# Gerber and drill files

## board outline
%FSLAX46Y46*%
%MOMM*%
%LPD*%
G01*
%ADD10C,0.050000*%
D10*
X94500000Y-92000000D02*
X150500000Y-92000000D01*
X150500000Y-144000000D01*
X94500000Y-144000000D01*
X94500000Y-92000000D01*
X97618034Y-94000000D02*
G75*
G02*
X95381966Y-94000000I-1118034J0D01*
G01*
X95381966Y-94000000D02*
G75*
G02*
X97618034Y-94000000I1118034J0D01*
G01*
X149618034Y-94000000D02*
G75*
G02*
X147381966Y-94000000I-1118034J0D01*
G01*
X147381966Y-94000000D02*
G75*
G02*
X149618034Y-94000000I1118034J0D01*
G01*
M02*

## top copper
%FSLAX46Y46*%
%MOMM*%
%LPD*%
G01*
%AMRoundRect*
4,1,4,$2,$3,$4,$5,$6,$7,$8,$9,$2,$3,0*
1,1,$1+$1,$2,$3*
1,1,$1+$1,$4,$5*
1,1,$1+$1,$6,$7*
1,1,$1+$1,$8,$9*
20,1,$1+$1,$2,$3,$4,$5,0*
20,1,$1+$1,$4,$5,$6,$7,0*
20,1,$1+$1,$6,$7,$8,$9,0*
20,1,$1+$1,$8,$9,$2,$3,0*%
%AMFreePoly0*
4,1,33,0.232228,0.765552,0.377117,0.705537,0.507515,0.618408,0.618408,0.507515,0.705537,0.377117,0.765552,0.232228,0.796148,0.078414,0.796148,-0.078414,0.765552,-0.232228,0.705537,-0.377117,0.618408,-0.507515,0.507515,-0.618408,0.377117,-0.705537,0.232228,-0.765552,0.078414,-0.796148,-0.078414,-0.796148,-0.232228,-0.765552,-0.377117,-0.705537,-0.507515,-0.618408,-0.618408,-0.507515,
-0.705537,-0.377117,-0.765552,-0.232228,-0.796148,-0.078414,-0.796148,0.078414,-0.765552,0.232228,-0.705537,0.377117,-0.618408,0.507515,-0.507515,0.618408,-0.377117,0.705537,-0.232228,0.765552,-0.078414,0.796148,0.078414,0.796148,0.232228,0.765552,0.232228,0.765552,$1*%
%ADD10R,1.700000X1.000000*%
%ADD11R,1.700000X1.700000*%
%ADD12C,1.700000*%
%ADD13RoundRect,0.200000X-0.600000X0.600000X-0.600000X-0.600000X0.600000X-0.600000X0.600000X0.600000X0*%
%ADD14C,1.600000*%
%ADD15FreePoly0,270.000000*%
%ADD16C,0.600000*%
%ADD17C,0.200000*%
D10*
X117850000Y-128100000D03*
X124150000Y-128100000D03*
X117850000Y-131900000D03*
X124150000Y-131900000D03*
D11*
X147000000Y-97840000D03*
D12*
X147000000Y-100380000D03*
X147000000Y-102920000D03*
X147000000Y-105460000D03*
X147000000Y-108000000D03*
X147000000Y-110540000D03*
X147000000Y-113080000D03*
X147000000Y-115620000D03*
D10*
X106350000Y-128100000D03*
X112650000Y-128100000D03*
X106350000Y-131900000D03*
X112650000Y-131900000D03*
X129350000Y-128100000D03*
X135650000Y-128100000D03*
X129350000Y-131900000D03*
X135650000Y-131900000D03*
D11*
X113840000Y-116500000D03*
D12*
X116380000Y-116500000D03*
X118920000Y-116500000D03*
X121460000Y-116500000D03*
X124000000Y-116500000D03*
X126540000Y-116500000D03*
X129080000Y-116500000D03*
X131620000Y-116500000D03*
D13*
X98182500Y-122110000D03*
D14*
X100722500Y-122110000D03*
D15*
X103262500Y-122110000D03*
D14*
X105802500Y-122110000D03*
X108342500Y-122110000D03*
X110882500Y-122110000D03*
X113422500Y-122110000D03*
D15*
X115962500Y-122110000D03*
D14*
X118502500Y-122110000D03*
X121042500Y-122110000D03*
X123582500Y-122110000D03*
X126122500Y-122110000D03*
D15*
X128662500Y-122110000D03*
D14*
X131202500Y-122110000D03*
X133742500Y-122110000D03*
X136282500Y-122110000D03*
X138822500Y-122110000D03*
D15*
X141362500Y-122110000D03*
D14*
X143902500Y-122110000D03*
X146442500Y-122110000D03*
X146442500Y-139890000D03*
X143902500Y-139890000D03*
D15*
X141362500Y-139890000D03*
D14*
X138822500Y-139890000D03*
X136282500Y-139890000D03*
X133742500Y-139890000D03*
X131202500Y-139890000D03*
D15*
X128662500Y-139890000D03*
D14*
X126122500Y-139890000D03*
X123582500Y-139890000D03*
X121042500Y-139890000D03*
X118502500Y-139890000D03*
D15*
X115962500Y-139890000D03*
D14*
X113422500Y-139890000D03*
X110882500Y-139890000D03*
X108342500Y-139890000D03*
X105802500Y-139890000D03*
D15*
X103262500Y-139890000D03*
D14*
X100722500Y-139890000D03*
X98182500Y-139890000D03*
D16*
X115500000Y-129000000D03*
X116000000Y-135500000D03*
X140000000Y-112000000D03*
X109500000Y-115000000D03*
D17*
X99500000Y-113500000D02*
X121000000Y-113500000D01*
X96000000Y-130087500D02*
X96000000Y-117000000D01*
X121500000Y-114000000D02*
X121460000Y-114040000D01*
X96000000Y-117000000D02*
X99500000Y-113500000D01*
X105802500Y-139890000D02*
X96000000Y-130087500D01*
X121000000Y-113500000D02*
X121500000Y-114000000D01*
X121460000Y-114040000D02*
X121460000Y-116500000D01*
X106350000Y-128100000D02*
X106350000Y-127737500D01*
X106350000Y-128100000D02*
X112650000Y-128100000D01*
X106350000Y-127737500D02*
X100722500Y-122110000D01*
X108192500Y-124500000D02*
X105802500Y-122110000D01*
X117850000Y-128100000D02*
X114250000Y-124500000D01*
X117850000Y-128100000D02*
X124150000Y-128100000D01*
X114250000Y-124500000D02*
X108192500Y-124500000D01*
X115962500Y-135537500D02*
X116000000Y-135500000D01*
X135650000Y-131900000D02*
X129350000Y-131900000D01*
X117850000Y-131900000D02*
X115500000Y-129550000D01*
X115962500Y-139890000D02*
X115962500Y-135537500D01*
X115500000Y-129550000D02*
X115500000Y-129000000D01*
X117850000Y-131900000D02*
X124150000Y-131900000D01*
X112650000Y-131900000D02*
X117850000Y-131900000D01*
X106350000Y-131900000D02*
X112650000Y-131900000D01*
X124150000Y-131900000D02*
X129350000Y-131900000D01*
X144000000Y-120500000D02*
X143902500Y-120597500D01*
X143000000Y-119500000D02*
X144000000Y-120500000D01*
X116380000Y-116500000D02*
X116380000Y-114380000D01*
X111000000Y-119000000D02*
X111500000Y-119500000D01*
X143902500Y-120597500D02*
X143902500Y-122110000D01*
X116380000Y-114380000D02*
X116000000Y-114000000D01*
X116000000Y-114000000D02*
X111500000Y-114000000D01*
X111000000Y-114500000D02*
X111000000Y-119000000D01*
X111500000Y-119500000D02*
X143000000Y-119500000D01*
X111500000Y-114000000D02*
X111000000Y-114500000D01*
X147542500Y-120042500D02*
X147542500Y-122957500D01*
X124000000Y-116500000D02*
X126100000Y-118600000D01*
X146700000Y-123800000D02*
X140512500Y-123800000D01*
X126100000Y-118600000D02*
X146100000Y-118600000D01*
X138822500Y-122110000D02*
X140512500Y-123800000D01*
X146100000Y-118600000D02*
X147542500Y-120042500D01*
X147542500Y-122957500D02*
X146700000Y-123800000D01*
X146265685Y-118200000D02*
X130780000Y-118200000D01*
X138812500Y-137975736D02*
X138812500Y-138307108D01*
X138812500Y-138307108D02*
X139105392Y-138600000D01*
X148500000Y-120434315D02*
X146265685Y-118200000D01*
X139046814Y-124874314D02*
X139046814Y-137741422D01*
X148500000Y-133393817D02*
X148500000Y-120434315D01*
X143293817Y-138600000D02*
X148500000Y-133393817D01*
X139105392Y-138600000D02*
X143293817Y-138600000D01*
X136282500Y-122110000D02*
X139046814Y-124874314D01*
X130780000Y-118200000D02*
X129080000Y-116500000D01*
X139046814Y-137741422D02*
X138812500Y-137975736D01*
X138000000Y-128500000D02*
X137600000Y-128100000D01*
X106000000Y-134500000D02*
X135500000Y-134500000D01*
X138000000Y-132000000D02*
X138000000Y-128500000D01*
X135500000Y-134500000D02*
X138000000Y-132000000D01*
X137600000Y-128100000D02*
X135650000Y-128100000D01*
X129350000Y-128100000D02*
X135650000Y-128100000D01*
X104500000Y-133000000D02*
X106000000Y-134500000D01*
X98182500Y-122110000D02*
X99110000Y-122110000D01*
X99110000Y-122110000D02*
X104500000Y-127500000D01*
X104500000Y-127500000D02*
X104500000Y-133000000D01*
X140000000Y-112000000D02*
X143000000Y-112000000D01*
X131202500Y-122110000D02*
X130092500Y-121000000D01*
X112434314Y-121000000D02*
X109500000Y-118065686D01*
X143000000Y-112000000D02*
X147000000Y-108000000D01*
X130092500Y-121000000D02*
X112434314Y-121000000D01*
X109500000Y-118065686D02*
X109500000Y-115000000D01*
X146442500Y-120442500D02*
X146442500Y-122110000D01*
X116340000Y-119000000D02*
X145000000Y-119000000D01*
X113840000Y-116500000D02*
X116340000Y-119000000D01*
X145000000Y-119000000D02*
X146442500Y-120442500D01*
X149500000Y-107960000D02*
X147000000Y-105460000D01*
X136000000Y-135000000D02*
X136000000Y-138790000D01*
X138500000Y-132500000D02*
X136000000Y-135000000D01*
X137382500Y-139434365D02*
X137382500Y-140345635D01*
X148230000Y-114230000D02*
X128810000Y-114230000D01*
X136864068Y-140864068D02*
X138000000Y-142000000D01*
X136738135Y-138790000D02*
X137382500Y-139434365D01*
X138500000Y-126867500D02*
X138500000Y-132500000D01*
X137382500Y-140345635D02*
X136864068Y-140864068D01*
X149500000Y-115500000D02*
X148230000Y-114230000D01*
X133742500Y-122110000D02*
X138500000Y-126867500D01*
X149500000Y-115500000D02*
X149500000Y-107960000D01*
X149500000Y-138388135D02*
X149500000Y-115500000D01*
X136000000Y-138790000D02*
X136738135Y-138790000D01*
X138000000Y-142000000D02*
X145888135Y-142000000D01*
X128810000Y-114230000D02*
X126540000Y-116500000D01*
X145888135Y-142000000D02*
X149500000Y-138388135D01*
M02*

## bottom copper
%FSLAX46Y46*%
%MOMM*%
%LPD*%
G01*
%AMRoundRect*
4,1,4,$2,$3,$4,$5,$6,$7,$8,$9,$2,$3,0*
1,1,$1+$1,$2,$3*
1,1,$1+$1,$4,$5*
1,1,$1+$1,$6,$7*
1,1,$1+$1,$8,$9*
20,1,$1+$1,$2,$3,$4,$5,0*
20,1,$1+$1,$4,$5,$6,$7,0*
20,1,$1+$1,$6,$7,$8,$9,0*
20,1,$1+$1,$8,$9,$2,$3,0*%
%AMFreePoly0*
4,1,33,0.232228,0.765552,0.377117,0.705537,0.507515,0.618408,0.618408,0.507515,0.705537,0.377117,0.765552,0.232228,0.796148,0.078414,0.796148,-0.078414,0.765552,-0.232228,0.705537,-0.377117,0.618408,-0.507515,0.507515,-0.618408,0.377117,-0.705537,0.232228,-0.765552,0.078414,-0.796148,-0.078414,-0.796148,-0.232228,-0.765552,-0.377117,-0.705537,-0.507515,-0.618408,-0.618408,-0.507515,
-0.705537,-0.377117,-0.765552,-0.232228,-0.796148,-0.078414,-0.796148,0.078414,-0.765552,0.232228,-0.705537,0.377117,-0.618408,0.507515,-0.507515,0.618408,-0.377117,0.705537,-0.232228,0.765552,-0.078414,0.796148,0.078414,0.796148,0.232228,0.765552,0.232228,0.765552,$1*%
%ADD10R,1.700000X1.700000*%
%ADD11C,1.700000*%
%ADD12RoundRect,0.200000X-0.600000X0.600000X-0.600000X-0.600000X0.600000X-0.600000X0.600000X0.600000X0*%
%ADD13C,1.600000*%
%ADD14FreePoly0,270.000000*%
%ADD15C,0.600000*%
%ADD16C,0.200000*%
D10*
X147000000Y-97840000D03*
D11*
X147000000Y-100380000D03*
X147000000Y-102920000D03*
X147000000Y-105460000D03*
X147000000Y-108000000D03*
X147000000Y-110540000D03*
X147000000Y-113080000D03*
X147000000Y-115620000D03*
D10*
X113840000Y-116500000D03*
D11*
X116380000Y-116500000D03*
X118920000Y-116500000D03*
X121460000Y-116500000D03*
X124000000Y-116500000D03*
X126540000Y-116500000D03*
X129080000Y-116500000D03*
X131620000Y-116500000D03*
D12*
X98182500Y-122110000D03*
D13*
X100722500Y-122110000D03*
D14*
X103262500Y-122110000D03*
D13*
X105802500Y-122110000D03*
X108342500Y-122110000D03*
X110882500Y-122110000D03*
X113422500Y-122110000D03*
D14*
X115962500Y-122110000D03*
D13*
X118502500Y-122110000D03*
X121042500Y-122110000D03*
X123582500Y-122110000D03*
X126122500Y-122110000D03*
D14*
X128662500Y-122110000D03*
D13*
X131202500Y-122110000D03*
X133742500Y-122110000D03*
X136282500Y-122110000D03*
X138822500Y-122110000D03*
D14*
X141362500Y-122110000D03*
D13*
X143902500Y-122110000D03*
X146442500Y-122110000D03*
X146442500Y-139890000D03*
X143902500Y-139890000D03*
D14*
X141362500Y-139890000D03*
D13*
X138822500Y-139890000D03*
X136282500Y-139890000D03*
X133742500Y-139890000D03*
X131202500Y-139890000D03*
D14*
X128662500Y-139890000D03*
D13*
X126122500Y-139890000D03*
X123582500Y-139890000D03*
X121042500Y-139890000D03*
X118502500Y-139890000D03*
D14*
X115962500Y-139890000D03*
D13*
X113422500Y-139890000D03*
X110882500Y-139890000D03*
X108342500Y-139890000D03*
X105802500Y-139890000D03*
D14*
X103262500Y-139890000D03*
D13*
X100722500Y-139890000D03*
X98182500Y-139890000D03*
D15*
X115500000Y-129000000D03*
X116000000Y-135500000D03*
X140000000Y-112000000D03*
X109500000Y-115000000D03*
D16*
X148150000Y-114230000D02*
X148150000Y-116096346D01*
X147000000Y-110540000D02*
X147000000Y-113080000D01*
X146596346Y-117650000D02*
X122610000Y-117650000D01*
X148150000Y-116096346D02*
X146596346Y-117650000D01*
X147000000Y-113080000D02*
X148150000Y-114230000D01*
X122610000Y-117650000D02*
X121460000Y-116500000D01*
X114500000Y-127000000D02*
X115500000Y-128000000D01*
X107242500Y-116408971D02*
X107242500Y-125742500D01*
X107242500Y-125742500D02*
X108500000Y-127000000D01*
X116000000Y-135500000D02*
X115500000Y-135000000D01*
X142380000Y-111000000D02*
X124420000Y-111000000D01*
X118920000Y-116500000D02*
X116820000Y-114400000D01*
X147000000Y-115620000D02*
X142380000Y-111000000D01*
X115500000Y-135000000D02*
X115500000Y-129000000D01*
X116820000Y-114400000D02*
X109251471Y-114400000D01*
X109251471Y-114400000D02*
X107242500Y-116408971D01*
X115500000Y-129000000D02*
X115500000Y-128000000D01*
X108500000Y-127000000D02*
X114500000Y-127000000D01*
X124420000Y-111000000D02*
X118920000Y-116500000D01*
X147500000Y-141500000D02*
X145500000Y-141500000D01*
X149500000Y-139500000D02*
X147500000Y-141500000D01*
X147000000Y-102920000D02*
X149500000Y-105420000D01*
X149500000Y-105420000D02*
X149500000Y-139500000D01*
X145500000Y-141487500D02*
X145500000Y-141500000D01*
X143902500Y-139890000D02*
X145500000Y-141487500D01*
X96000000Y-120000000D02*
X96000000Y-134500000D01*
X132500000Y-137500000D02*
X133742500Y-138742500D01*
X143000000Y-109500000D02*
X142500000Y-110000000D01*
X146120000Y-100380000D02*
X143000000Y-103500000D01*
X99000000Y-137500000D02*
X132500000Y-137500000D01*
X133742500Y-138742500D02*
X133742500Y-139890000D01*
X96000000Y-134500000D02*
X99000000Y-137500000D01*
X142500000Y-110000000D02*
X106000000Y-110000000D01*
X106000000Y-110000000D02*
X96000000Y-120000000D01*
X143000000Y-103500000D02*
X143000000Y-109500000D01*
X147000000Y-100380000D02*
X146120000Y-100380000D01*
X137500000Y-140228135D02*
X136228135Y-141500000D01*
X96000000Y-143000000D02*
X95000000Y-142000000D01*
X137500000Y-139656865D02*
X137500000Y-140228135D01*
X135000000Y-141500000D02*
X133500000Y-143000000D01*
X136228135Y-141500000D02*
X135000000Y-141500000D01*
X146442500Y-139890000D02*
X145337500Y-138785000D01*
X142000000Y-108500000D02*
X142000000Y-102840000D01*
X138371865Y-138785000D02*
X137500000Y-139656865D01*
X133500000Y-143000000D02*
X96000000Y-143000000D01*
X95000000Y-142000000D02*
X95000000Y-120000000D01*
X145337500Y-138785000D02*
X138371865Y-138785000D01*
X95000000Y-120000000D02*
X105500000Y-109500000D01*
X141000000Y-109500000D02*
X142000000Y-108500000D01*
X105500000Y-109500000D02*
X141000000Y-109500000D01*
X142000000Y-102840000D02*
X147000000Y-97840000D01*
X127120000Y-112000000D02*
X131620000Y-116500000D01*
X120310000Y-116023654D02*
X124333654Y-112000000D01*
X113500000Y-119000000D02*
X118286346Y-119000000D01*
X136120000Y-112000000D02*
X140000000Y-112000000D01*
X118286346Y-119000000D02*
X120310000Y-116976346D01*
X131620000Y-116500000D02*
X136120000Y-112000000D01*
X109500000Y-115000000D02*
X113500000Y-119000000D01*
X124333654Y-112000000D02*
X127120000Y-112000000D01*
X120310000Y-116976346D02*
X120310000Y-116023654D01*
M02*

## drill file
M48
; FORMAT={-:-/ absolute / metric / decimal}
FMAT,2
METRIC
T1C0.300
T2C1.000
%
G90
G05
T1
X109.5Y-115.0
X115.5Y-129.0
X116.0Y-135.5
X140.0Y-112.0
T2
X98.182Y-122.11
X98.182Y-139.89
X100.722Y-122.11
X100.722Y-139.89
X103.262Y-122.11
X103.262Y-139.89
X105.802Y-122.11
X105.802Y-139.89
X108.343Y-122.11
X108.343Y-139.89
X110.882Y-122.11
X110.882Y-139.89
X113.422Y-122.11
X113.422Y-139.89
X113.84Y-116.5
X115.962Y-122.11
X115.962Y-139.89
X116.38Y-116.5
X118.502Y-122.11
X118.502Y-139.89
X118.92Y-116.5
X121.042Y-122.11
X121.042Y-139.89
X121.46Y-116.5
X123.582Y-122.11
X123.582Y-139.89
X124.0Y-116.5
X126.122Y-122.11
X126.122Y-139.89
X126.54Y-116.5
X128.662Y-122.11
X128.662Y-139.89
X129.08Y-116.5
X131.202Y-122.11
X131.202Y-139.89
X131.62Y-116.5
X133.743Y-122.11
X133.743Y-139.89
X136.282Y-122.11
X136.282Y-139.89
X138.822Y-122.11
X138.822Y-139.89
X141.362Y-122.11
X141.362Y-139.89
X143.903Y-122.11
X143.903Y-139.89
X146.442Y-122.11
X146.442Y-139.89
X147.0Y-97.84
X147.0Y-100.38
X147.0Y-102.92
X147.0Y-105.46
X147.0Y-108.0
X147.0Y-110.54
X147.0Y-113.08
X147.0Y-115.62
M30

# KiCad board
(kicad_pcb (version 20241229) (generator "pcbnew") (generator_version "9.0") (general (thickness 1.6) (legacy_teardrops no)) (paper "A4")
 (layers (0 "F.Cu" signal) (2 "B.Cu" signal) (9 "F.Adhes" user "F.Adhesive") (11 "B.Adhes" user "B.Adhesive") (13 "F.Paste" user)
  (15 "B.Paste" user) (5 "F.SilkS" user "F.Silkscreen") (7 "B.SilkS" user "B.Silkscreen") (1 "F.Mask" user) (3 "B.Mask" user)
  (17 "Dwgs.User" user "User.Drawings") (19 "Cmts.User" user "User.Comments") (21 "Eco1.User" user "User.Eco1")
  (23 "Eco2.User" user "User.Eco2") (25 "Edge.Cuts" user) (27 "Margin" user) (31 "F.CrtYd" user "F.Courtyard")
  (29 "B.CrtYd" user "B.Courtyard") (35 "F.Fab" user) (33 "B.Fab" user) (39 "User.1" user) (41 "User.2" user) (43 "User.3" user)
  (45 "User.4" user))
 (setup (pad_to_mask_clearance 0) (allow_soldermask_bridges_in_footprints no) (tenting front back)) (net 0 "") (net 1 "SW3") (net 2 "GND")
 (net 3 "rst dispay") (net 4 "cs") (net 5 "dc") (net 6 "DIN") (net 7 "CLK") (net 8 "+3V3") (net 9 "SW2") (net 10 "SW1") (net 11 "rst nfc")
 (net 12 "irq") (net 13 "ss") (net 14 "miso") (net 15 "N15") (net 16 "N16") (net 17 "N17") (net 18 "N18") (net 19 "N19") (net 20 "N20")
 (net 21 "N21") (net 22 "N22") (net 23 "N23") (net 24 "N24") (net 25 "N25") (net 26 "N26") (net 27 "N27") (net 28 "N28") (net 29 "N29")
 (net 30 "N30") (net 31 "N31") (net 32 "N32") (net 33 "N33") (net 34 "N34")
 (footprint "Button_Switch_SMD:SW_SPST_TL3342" (layer "F.Cu") (at 121 130)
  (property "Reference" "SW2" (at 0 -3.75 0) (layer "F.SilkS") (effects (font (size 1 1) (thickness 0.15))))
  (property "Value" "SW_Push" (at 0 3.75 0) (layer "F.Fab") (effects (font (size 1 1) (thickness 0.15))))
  (pad "1" smd rect (at -3.15 -1.9) (size 1.7 1) (layers "F.Cu" "F.Mask" "F.Paste") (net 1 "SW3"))
  (pad "1" smd rect (at 3.15 -1.9) (size 1.7 1) (layers "F.Cu" "F.Mask" "F.Paste") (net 1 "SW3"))
  (pad "2" smd rect (at -3.15 1.9) (size 1.7 1) (layers "F.Cu" "F.Mask" "F.Paste") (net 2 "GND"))
  (pad "2" smd rect (at 3.15 1.9) (size 1.7 1) (layers "F.Cu" "F.Mask" "F.Paste") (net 2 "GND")))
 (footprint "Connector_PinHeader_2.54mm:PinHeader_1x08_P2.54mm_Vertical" (layer "F.Cu") (at 147 97.84)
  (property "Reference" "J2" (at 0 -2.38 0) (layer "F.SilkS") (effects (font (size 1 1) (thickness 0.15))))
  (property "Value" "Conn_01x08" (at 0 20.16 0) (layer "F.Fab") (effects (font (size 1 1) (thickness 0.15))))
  (pad "1" thru_hole rect (at 0 0) (size 1.7 1.7) (drill 1) (layers "*.Cu" "*.Mask") (remove_unused_layers no) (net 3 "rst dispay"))
  (pad "2" thru_hole circle (at 0 2.54) (size 1.7 1.7) (drill 1) (layers "*.Cu" "*.Mask") (remove_unused_layers no) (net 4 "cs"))
  (pad "3" thru_hole circle (at 0 5.08) (size 1.7 1.7) (drill 1) (layers "*.Cu" "*.Mask") (remove_unused_layers no) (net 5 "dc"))
  (pad "4" thru_hole circle (at 0 7.62) (size 1.7 1.7) (drill 1) (layers "*.Cu" "*.Mask") (remove_unused_layers no) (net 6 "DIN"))
  (pad "5" thru_hole circle (at 0 10.16) (size 1.7 1.7) (drill 1) (layers "*.Cu" "*.Mask") (remove_unused_layers no) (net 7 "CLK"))
  (pad "6" thru_hole circle (at 0 12.7) (size 1.7 1.7) (drill 1) (layers "*.Cu" "*.Mask") (remove_unused_layers no) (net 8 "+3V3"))
  (pad "7" thru_hole circle (at 0 15.24) (size 1.7 1.7) (drill 1) (layers "*.Cu" "*.Mask") (remove_unused_layers no) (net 8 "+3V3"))
  (pad "8" thru_hole circle (at 0 17.78) (size 1.7 1.7) (drill 1) (layers "*.Cu" "*.Mask") (remove_unused_layers no) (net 2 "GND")))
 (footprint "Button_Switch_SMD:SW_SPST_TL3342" (layer "F.Cu") (at 109.5 130)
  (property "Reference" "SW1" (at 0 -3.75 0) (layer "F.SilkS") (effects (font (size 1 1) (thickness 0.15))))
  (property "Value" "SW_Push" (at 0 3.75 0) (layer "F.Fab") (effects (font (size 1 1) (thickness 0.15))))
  (pad "1" smd rect (at -3.15 -1.9) (size 1.7 1) (layers "F.Cu" "F.Mask" "F.Paste") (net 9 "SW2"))
  (pad "1" smd rect (at 3.15 -1.9) (size 1.7 1) (layers "F.Cu" "F.Mask" "F.Paste") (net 9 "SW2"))
  (pad "2" smd rect (at -3.15 1.9) (size 1.7 1) (layers "F.Cu" "F.Mask" "F.Paste") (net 2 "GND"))
  (pad "2" smd rect (at 3.15 1.9) (size 1.7 1) (layers "F.Cu" "F.Mask" "F.Paste") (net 2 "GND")))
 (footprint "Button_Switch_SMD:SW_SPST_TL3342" (layer "F.Cu") (at 132.5 130)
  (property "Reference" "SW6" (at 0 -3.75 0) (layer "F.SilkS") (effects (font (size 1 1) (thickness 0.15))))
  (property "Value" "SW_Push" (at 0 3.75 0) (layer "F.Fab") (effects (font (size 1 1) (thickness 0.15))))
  (pad "1" smd rect (at -3.15 -1.9) (size 1.7 1) (layers "F.Cu" "F.Mask" "F.Paste") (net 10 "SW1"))
  (pad "1" smd rect (at 3.15 -1.9) (size 1.7 1) (layers "F.Cu" "F.Mask" "F.Paste") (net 10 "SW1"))
  (pad "2" smd rect (at -3.15 1.9) (size 1.7 1) (layers "F.Cu" "F.Mask" "F.Paste") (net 2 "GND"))
  (pad "2" smd rect (at 3.15 1.9) (size 1.7 1) (layers "F.Cu" "F.Mask" "F.Paste") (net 2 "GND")))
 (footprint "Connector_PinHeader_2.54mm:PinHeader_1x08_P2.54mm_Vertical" (layer "F.Cu") (at 113.84 116.5 90)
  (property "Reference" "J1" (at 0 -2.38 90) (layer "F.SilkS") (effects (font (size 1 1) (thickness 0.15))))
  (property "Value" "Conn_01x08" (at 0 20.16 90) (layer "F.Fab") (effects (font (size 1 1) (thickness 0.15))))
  (pad "1" thru_hole rect (at 0 0 90) (size 1.7 1.7) (drill 1) (layers "*.Cu" "*.Mask") (remove_unused_layers no) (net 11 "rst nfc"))
  (pad "2" thru_hole circle (at 0 2.54 90) (size 1.7 1.7) (drill 1) (layers "*.Cu" "*.Mask") (remove_unused_layers no) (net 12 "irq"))
  (pad "3" thru_hole circle (at 0 5.08 90) (size 1.7 1.7) (drill 1) (layers "*.Cu" "*.Mask") (remove_unused_layers no) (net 2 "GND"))
  (pad "4" thru_hole circle (at 0 7.62 90) (size 1.7 1.7) (drill 1) (layers "*.Cu" "*.Mask") (remove_unused_layers no) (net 8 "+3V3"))
  (pad "5" thru_hole circle (at 0 10.16 90) (size 1.7 1.7) (drill 1) (layers "*.Cu" "*.Mask") (remove_unused_layers no) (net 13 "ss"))
  (pad "6" thru_hole circle (at 0 12.7 90) (size 1.7 1.7) (drill 1) (layers "*.Cu" "*.Mask") (remove_unused_layers no) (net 6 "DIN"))
  (pad "7" thru_hole circle (at 0 15.24 90) (size 1.7 1.7) (drill 1) (layers "*.Cu" "*.Mask") (remove_unused_layers no) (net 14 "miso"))
  (pad "8" thru_hole circle (at 0 17.78 90) (size 1.7 1.7) (drill 1) (layers "*.Cu" "*.Mask") (remove_unused_layers no) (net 7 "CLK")))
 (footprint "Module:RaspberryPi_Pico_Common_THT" (layer "B.Cu") (at 98.1825 122.11 -90)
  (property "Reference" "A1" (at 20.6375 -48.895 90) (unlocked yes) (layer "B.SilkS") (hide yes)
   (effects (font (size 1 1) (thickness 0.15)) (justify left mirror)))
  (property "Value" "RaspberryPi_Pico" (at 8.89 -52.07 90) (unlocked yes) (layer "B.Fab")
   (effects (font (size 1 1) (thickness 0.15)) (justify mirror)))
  (pad "1" thru_hole roundrect (at 0 0 270) (size 1.6 1.6) (drill 1) (layers "*.Cu" "*.Mask") (remove_unused_layers no)
   (roundrect_rratio 0.125) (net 10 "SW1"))
  (pad "2" thru_hole circle (at 0 -2.54 270) (size 1.6 1.6) (drill 1) (layers "*.Cu" "*.Mask") (remove_unused_layers no) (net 9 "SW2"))
  (pad "3" thru_hole custom (at 0 -5.08 270) (size 1.6 1.6) (drill 1) (layers "*.Cu" "*.Mask") (remove_unused_layers no) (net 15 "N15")
   (options (clearance outline) (anchor circle)) (primitives))
  (pad "4" thru_hole circle (at 0 -7.62 270) (size 1.6 1.6) (drill 1) (layers "*.Cu" "*.Mask") (remove_unused_layers no) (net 1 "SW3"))
  (pad "5" thru_hole circle (at 0 -10.16 270) (size 1.6 1.6) (drill 1) (layers "*.Cu" "*.Mask") (remove_unused_layers no) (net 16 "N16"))
  (pad "6" thru_hole circle (at 0 -12.7 270) (size 1.6 1.6) (drill 1) (layers "*.Cu" "*.Mask") (remove_unused_layers no) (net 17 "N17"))
  (pad "7" thru_hole circle (at 0 -15.24 270) (size 1.6 1.6) (drill 1) (layers "*.Cu" "*.Mask") (remove_unused_layers no) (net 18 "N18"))
  (pad "8" thru_hole custom (at 0 -17.78 270) (size 1.6 1.6) (drill 1) (layers "*.Cu" "*.Mask") (remove_unused_layers no) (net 15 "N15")
   (options (clearance outline) (anchor circle)) (primitives))
  (pad "9" thru_hole circle (at 0 -20.32 270) (size 1.6 1.6) (drill 1) (layers "*.Cu" "*.Mask") (remove_unused_layers no) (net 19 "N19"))
  (pad "10" thru_hole circle (at 0 -22.86 270) (size 1.6 1.6) (drill 1) (layers "*.Cu" "*.Mask") (remove_unused_layers no) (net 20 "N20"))
  (pad "11" thru_hole circle (at 0 -25.4 270) (size 1.6 1.6) (drill 1) (layers "*.Cu" "*.Mask") (remove_unused_layers no) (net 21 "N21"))
  (pad "12" thru_hole circle (at 0 -27.94 270) (size 1.6 1.6) (drill 1) (layers "*.Cu" "*.Mask") (remove_unused_layers no) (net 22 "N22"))
  (pad "13" thru_hole custom (at 0 -30.48 270) (size 1.6 1.6) (drill 1) (layers "*.Cu" "*.Mask") (remove_unused_layers no) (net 15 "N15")
   (options (clearance outline) (anchor circle)) (primitives))
  (pad "14" thru_hole circle (at 0 -33.02 270) (size 1.6 1.6) (drill 1) (layers "*.Cu" "*.Mask") (remove_unused_layers no) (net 7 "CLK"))
  (pad "15" thru_hole circle (at 0 -35.56 270) (size 1.6 1.6) (drill 1) (layers "*.Cu" "*.Mask") (remove_unused_layers no) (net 6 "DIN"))
  (pad "16" thru_hole circle (at 0 -38.1 270) (size 1.6 1.6) (drill 1) (layers "*.Cu" "*.Mask") (remove_unused_layers no) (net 14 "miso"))
  (pad "17" thru_hole circle (at 0 -40.64 270) (size 1.6 1.6) (drill 1) (layers "*.Cu" "*.Mask") (remove_unused_layers no) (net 13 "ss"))
  (pad "18" thru_hole custom (at 0 -43.18 270) (size 1.6 1.6) (drill 1) (layers "*.Cu" "*.Mask") (remove_unused_layers no) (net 15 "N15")
   (options (clearance outline) (anchor circle)) (primitives))
  (pad "19" thru_hole circle (at 0 -45.72 270) (size 1.6 1.6) (drill 1) (layers "*.Cu" "*.Mask") (remove_unused_layers no) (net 12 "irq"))
  (pad "20" thru_hole circle (at 0 -48.26 270) (size 1.6 1.6) (drill 1) (layers "*.Cu" "*.Mask") (remove_unused_layers no)
   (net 11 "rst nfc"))
  (pad "21" thru_hole circle (at 17.78 -48.26 270) (size 1.6 1.6) (drill 1) (layers "*.Cu" "*.Mask") (remove_unused_layers no)
   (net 3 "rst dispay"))
  (pad "22" thru_hole circle (at 17.78 -45.72 270) (size 1.6 1.6) (drill 1) (layers "*.Cu" "*.Mask") (remove_unused_layers no) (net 5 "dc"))
  (pad "23" thru_hole custom (at 17.78 -43.18 270) (size 1.6 1.6) (drill 1) (layers "*.Cu" "*.Mask") (remove_unused_layers no)
   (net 15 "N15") (options (clearance outline) (anchor circle)) (primitives))
  (pad "24" thru_hole circle (at 17.78 -40.64 270) (size 1.6 1.6) (drill 1) (layers "*.Cu" "*.Mask") (remove_unused_layers no)
   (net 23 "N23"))
  (pad "25" thru_hole circle (at 17.78 -38.1 270) (size 1.6 1.6) (drill 1) (layers "*.Cu" "*.Mask") (remove_unused_layers no) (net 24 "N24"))
  (pad "26" thru_hole circle (at 17.78 -35.56 270) (size 1.6 1.6) (drill 1) (layers "*.Cu" "*.Mask") (remove_unused_layers no) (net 4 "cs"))
  (pad "27" thru_hole circle (at 17.78 -33.02 270) (size 1.6 1.6) (drill 1) (layers "*.Cu" "*.Mask") (remove_unused_layers no)
   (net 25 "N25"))
  (pad "28" thru_hole custom (at 17.78 -30.48 270) (size 1.6 1.6) (drill 1) (layers "*.Cu" "*.Mask") (remove_unused_layers no)
   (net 15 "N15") (options (clearance outline) (anchor circle)) (primitives))
  (pad "29" thru_hole circle (at 17.78 -27.94 270) (size 1.6 1.6) (drill 1) (layers "*.Cu" "*.Mask") (remove_unused_layers no)
   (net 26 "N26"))
  (pad "30" thru_hole circle (at 17.78 -25.4 270) (size 1.6 1.6) (drill 1) (layers "*.Cu" "*.Mask") (remove_unused_layers no) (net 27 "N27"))
  (pad "31" thru_hole circle (at 17.78 -22.86 270) (size 1.6 1.6) (drill 1) (layers "*.Cu" "*.Mask") (remove_unused_layers no)
   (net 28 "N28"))
  (pad "32" thru_hole circle (at 17.78 -20.32 270) (size 1.6 1.6) (drill 1) (layers "*.Cu" "*.Mask") (remove_unused_layers no)
   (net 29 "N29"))
  (pad "33" thru_hole custom (at 17.78 -17.78 270) (size 1.6 1.6) (drill 1) (layers "*.Cu" "*.Mask") (remove_unused_layers no) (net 2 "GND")
   (options (clearance outline) (anchor circle)) (primitives))
  (pad "34" thru_hole circle (at 17.78 -15.24 270) (size 1.6 1.6) (drill 1) (layers "*.Cu" "*.Mask") (remove_unused_layers no)
   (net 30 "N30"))
  (pad "35" thru_hole circle (at 17.78 -12.7 270) (size 1.6 1.6) (drill 1) (layers "*.Cu" "*.Mask") (remove_unused_layers no) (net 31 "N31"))
  (pad "36" thru_hole circle (at 17.78 -10.16 270) (size 1.6 1.6) (drill 1) (layers "*.Cu" "*.Mask") (remove_unused_layers no)
   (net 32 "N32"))
  (pad "37" thru_hole circle (at 17.78 -7.62 270) (size 1.6 1.6) (drill 1) (layers "*.Cu" "*.Mask") (remove_unused_layers no) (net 8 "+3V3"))
  (pad "38" thru_hole custom (at 17.78 -5.08 270) (size 1.6 1.6) (drill 1) (layers "*.Cu" "*.Mask") (remove_unused_layers no) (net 15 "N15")
   (options (clearance outline) (anchor circle)) (primitives))
  (pad "39" thru_hole circle (at 17.78 -2.54 270) (size 1.6 1.6) (drill 1) (layers "*.Cu" "*.Mask") (remove_unused_layers no) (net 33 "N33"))
  (pad "40" thru_hole circle (at 17.78 0 270) (size 1.6 1.6) (drill 1) (layers "*.Cu" "*.Mask") (remove_unused_layers no) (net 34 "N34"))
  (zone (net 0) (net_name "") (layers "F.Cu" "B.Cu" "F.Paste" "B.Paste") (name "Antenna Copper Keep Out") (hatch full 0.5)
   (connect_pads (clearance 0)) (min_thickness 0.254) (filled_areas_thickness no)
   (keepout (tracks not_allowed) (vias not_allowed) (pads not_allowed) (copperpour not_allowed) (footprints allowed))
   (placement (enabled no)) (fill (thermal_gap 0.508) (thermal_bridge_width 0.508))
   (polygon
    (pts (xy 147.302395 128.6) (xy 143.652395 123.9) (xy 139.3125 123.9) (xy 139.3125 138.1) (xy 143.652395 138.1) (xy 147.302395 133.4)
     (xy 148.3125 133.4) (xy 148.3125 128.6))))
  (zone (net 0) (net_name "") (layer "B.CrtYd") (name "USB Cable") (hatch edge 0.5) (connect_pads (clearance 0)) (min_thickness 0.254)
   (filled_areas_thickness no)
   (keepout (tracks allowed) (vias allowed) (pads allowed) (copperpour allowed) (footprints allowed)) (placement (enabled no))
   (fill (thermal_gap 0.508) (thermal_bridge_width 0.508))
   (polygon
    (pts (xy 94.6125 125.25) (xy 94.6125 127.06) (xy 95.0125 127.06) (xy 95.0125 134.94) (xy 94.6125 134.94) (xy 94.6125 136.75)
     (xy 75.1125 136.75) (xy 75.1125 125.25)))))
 (gr_rect (start 94.5 92) (end 150.5 144) (stroke (width 0.05) (type default)) (fill no) (layer "Edge.Cuts"))
 (gr_circle (center 96.5 94) (end 97.5 94.5) (stroke (width 0.05) (type default)) (fill no) (layer "Edge.Cuts"))
 (gr_circle (center 148.5 94) (end 149.5 94.5) (stroke (width 0.05) (type default)) (fill no) (layer "Edge.Cuts"))
 (segment (start 99.5 113.5) (end 121 113.5) (width 0.2) (layer "F.Cu") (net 8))
 (segment (start 96 130.0875) (end 96 117) (width 0.2) (layer "F.Cu") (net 8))
 (segment (start 121.5 114) (end 121.46 114.04) (width 0.2) (layer "F.Cu") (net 8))
 (segment (start 96 117) (end 99.5 113.5) (width 0.2) (layer "F.Cu") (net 8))
 (segment (start 105.8025 139.89) (end 96 130.0875) (width 0.2) (layer "F.Cu") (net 8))
 (segment (start 121 113.5) (end 121.5 114) (width 0.2) (layer "F.Cu") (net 8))
 (segment (start 121.46 114.04) (end 121.46 116.5) (width 0.2) (layer "F.Cu") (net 8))
 (segment (start 148.15 114.23) (end 148.15 116.096346) (width 0.2) (layer "B.Cu") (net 8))
 (segment (start 147 110.54) (end 147 113.08) (width 0.2) (layer "B.Cu") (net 8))
 (segment (start 146.596346 117.65) (end 122.61 117.65) (width 0.2) (layer "B.Cu") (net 8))
 (segment (start 148.15 116.096346) (end 146.596346 117.65) (width 0.2) (layer "B.Cu") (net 8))
 (segment (start 147 113.08) (end 148.15 114.23) (width 0.2) (layer "B.Cu") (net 8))
 (segment (start 122.61 117.65) (end 121.46 116.5) (width 0.2) (layer "B.Cu") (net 8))
 (segment (start 106.35 128.1) (end 106.35 127.7375) (width 0.2) (layer "F.Cu") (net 9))
 (segment (start 106.35 128.1) (end 112.65 128.1) (width 0.2) (layer "F.Cu") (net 9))
 (segment (start 106.35 127.7375) (end 100.7225 122.11) (width 0.2) (layer "F.Cu") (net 9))
 (segment (start 108.1925 124.5) (end 105.8025 122.11) (width 0.2) (layer "F.Cu") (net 1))
 (segment (start 117.85 128.1) (end 114.25 124.5) (width 0.2) (layer "F.Cu") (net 1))
 (segment (start 117.85 128.1) (end 124.15 128.1) (width 0.2) (layer "F.Cu") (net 1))
 (segment (start 114.25 124.5) (end 108.1925 124.5) (width 0.2) (layer "F.Cu") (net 1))
 (segment (start 115.9625 135.5375) (end 116 135.5) (width 0.2) (layer "F.Cu") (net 2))
 (segment (start 135.65 131.9) (end 129.35 131.9) (width 0.2) (layer "F.Cu") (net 2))
 (segment (start 117.85 131.9) (end 115.5 129.55) (width 0.2) (layer "F.Cu") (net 2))
 (segment (start 115.9625 139.89) (end 115.9625 135.5375) (width 0.2) (layer "F.Cu") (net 2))
 (segment (start 115.5 129.55) (end 115.5 129) (width 0.2) (layer "F.Cu") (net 2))
 (segment (start 117.85 131.9) (end 124.15 131.9) (width 0.2) (layer "F.Cu") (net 2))
 (segment (start 112.65 131.9) (end 117.85 131.9) (width 0.2) (layer "F.Cu") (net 2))
 (segment (start 106.35 131.9) (end 112.65 131.9) (width 0.2) (layer "F.Cu") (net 2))
 (segment (start 124.15 131.9) (end 129.35 131.9) (width 0.2) (layer "F.Cu") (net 2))
 (via (at 115.5 129) (size 0.6) (drill 0.3) (layers "F.Cu" "B.Cu") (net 2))
 (via (at 116 135.5) (size 0.6) (drill 0.3) (layers "F.Cu" "B.Cu") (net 2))
 (segment (start 114.5 127) (end 115.5 128) (width 0.2) (layer "B.Cu") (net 2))
 (segment (start 107.2425 116.408971) (end 107.2425 125.7425) (width 0.2) (layer "B.Cu") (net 2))
 (segment (start 107.2425 125.7425) (end 108.5 127) (width 0.2) (layer "B.Cu") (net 2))
 (segment (start 116 135.5) (end 115.5 135) (width 0.2) (layer "B.Cu") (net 2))
 (segment (start 142.38 111) (end 124.42 111) (width 0.2) (layer "B.Cu") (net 2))
 (segment (start 118.92 116.5) (end 116.82 114.4) (width 0.2) (layer "B.Cu") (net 2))
 (segment (start 147 115.62) (end 142.38 111) (width 0.2) (layer "B.Cu") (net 2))
 (segment (start 115.5 135) (end 115.5 129) (width 0.2) (layer "B.Cu") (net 2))
 (segment (start 116.82 114.4) (end 109.251471 114.4) (width 0.2) (layer "B.Cu") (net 2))
 (segment (start 109.251471 114.4) (end 107.2425 116.408971) (width 0.2) (layer "B.Cu") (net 2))
 (segment (start 115.5 129) (end 115.5 128) (width 0.2) (layer "B.Cu") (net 2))
 (segment (start 108.5 127) (end 114.5 127) (width 0.2) (layer "B.Cu") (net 2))
 (segment (start 124.42 111) (end 118.92 116.5) (width 0.2) (layer "B.Cu") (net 2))
 (segment (start 144 120.5) (end 143.9025 120.5975) (width 0.2) (layer "F.Cu") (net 12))
 (segment (start 143 119.5) (end 144 120.5) (width 0.2) (layer "F.Cu") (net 12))
 (segment (start 116.38 116.5) (end 116.38 114.38) (width 0.2) (layer "F.Cu") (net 12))
 (segment (start 111 119) (end 111.5 119.5) (width 0.2) (layer "F.Cu") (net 12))
 (segment (start 143.9025 120.5975) (end 143.9025 122.11) (width 0.2) (layer "F.Cu") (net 12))
 (segment (start 116.38 114.38) (end 116 114) (width 0.2) (layer "F.Cu") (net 12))
 (segment (start 116 114) (end 111.5 114) (width 0.2) (layer "F.Cu") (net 12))
 (segment (start 111 114.5) (end 111 119) (width 0.2) (layer "F.Cu") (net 12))
 (segment (start 111.5 119.5) (end 143 119.5) (width 0.2) (layer "F.Cu") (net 12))
 (segment (start 111.5 114) (end 111 114.5) (width 0.2) (layer "F.Cu") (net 12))
 (segment (start 147.5 141.5) (end 145.5 141.5) (width 0.2) (layer "B.Cu") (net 5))
 (segment (start 149.5 139.5) (end 147.5 141.5) (width 0.2) (layer "B.Cu") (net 5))
 (segment (start 147 102.92) (end 149.5 105.42) (width 0.2) (layer "B.Cu") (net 5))
 (segment (start 149.5 105.42) (end 149.5 139.5) (width 0.2) (layer "B.Cu") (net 5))
 (segment (start 145.5 141.4875) (end 145.5 141.5) (width 0.2) (layer "B.Cu") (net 5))
 (segment (start 143.9025 139.89) (end 145.5 141.4875) (width 0.2) (layer "B.Cu") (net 5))
 (segment (start 147.5425 120.0425) (end 147.5425 122.9575) (width 0.2) (layer "F.Cu") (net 13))
 (segment (start 124 116.5) (end 126.1 118.6) (width 0.2) (layer "F.Cu") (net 13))
 (segment (start 146.7 123.8) (end 140.5125 123.8) (width 0.2) (layer "F.Cu") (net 13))
 (segment (start 126.1 118.6) (end 146.1 118.6) (width 0.2) (layer "F.Cu") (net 13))
 (segment (start 138.8225 122.11) (end 140.5125 123.8) (width 0.2) (layer "F.Cu") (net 13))
 (segment (start 146.1 118.6) (end 147.5425 120.0425) (width 0.2) (layer "F.Cu") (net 13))
 (segment (start 147.5425 122.9575) (end 146.7 123.8) (width 0.2) (layer "F.Cu") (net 13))
 (segment (start 146.265685 118.2) (end 130.78 118.2) (width 0.2) (layer "F.Cu") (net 14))
 (segment (start 138.8125 137.975736) (end 138.8125 138.307108) (width 0.2) (layer "F.Cu") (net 14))
 (segment (start 138.8125 138.307108) (end 139.105392 138.6) (width 0.2) (layer "F.Cu") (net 14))
 (segment (start 148.5 120.434315) (end 146.265685 118.2) (width 0.2) (layer "F.Cu") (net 14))
 (segment (start 139.046814 124.874314) (end 139.046814 137.741422) (width 0.2) (layer "F.Cu") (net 14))
 (segment (start 148.5 133.393817) (end 148.5 120.434315) (width 0.2) (layer "F.Cu") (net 14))
 (segment (start 143.293817 138.6) (end 148.5 133.393817) (width 0.2) (layer "F.Cu") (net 14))
 (segment (start 139.105392 138.6) (end 143.293817 138.6) (width 0.2) (layer "F.Cu") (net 14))
 (segment (start 136.2825 122.11) (end 139.046814 124.874314) (width 0.2) (layer "F.Cu") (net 14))
 (segment (start 130.78 118.2) (end 129.08 116.5) (width 0.2) (layer "F.Cu") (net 14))
 (segment (start 139.046814 137.741422) (end 138.8125 137.975736) (width 0.2) (layer "F.Cu") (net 14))
 (segment (start 96 120) (end 96 134.5) (width 0.2) (layer "B.Cu") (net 4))
 (segment (start 132.5 137.5) (end 133.7425 138.7425) (width 0.2) (layer "B.Cu") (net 4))
 (segment (start 143 109.5) (end 142.5 110) (width 0.2) (layer "B.Cu") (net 4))
 (segment (start 146.12 100.38) (end 143 103.5) (width 0.2) (layer "B.Cu") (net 4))
 (segment (start 99 137.5) (end 132.5 137.5) (width 0.2) (layer "B.Cu") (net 4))
 (segment (start 133.7425 138.7425) (end 133.7425 139.89) (width 0.2) (layer "B.Cu") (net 4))
 (segment (start 96 134.5) (end 99 137.5) (width 0.2) (layer "B.Cu") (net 4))
 (segment (start 142.5 110) (end 106 110) (width 0.2) (layer "B.Cu") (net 4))
 (segment (start 106 110) (end 96 120) (width 0.2) (layer "B.Cu") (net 4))
 (segment (start 143 103.5) (end 143 109.5) (width 0.2) (layer "B.Cu") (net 4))
 (segment (start 147 100.38) (end 146.12 100.38) (width 0.2) (layer "B.Cu") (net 4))
 (segment (start 138 128.5) (end 137.6 128.1) (width 0.2) (layer "F.Cu") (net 10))
 (segment (start 106 134.5) (end 135.5 134.5) (width 0.2) (layer "F.Cu") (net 10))
 (segment (start 138 132) (end 138 128.5) (width 0.2) (layer "F.Cu") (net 10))
 (segment (start 135.5 134.5) (end 138 132) (width 0.2) (layer "F.Cu") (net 10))
 (segment (start 137.6 128.1) (end 135.65 128.1) (width 0.2) (layer "F.Cu") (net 10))
 (segment (start 129.35 128.1) (end 135.65 128.1) (width 0.2) (layer "F.Cu") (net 10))
 (segment (start 104.5 133) (end 106 134.5) (width 0.2) (layer "F.Cu") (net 10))
 (segment (start 98.1825 122.11) (end 99.11 122.11) (width 0.2) (layer "F.Cu") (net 10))
 (segment (start 99.11 122.11) (end 104.5 127.5) (width 0.2) (layer "F.Cu") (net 10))
 (segment (start 104.5 127.5) (end 104.5 133) (width 0.2) (layer "F.Cu") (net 10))
 (segment (start 137.5 140.228135) (end 136.228135 141.5) (width 0.2) (layer "B.Cu") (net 3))
 (segment (start 96 143) (end 95 142) (width 0.2) (layer "B.Cu") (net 3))
 (segment (start 137.5 139.656865) (end 137.5 140.228135) (width 0.2) (layer "B.Cu") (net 3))
 (segment (start 135 141.5) (end 133.5 143) (width 0.2) (layer "B.Cu") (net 3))
 (segment (start 136.228135 141.5) (end 135 141.5) (width 0.2) (layer "B.Cu") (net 3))
 (segment (start 146.4425 139.89) (end 145.3375 138.785) (width 0.2) (layer "B.Cu") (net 3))
 (segment (start 142 108.5) (end 142 102.84) (width 0.2) (layer "B.Cu") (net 3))
 (segment (start 138.371865 138.785) (end 137.5 139.656865) (width 0.2) (layer "B.Cu") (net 3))
 (segment (start 133.5 143) (end 96 143) (width 0.2) (layer "B.Cu") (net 3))
 (segment (start 95 142) (end 95 120) (width 0.2) (layer "B.Cu") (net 3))
 (segment (start 145.3375 138.785) (end 138.371865 138.785) (width 0.2) (layer "B.Cu") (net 3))
 (segment (start 95 120) (end 105.5 109.5) (width 0.2) (layer "B.Cu") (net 3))
 (segment (start 141 109.5) (end 142 108.5) (width 0.2) (layer "B.Cu") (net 3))
 (segment (start 105.5 109.5) (end 141 109.5) (width 0.2) (layer "B.Cu") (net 3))
 (segment (start 142 102.84) (end 147 97.84) (width 0.2) (layer "B.Cu") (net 3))
 (segment (start 140 112) (end 143 112) (width 0.2) (layer "F.Cu") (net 7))
 (segment (start 131.2025 122.11) (end 130.0925 121) (width 0.2) (layer "F.Cu") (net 7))
 (segment (start 112.434314 121) (end 109.5 118.065686) (width 0.2) (layer "F.Cu") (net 7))
 (segment (start 143 112) (end 147 108) (width 0.2) (layer "F.Cu") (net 7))
 (segment (start 130.0925 121) (end 112.434314 121) (width 0.2) (layer "F.Cu") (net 7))
 (segment (start 109.5 118.065686) (end 109.5 115) (width 0.2) (layer "F.Cu") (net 7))
 (via (at 140 112) (size 0.6) (drill 0.3) (layers "F.Cu" "B.Cu") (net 7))
 (via (at 109.5 115) (size 0.6) (drill 0.3) (layers "F.Cu" "B.Cu") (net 7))
 (segment (start 127.12 112) (end 131.62 116.5) (width 0.2) (layer "B.Cu") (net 7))
 (segment (start 120.31 116.023654) (end 124.333654 112) (width 0.2) (layer "B.Cu") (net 7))
 (segment (start 113.5 119) (end 118.286346 119) (width 0.2) (layer "B.Cu") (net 7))
 (segment (start 136.12 112) (end 140 112) (width 0.2) (layer "B.Cu") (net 7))
 (segment (start 118.286346 119) (end 120.31 116.976346) (width 0.2) (layer "B.Cu") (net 7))
 (segment (start 131.62 116.5) (end 136.12 112) (width 0.2) (layer "B.Cu") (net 7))
 (segment (start 109.5 115) (end 113.5 119) (width 0.2) (layer "B.Cu") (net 7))
 (segment (start 124.333654 112) (end 127.12 112) (width 0.2) (layer "B.Cu") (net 7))
 (segment (start 120.31 116.976346) (end 120.31 116.023654) (width 0.2) (layer "B.Cu") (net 7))
 (segment (start 146.4425 120.4425) (end 146.4425 122.11) (width 0.2) (layer "F.Cu") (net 11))
 (segment (start 116.34 119) (end 145 119) (width 0.2) (layer "F.Cu") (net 11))
 (segment (start 113.84 116.5) (end 116.34 119) (width 0.2) (layer "F.Cu") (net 11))
 (segment (start 145 119) (end 146.4425 120.4425) (width 0.2) (layer "F.Cu") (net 11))
 (segment (start 149.5 107.96) (end 147 105.46) (width 0.2) (layer "F.Cu") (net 6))
 (segment (start 136 135) (end 136 138.79) (width 0.2) (layer "F.Cu") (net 6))
 (segment (start 138.5 132.5) (end 136 135) (width 0.2) (layer "F.Cu") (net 6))
 (segment (start 137.3825 139.434365) (end 137.3825 140.345635) (width 0.2) (layer "F.Cu") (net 6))
 (segment (start 148.23 114.23) (end 128.81 114.23) (width 0.2) (layer "F.Cu") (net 6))
 (segment (start 136.864068 140.864068) (end 138 142) (width 0.2) (layer "F.Cu") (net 6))
 (segment (start 136.738135 138.79) (end 137.3825 139.434365) (width 0.2) (layer "F.Cu") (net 6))
 (segment (start 138.5 126.8675) (end 138.5 132.5) (width 0.2) (layer "F.Cu") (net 6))
 (segment (start 137.3825 140.345635) (end 136.864068 140.864068) (width 0.2) (layer "F.Cu") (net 6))
 (segment (start 149.5 115.5) (end 148.23 114.23) (width 0.2) (layer "F.Cu") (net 6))
 (segment (start 133.7425 122.11) (end 138.5 126.8675) (width 0.2) (layer "F.Cu") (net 6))
 (segment (start 149.5 115.5) (end 149.5 107.96) (width 0.2) (layer "F.Cu") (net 6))
 (segment (start 149.5 138.388135) (end 149.5 115.5) (width 0.2) (layer "F.Cu") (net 6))
 (segment (start 136 138.79) (end 136.738135 138.79) (width 0.2) (layer "F.Cu") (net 6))
 (segment (start 138 142) (end 145.888135 142) (width 0.2) (layer "F.Cu") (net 6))
 (segment (start 128.81 114.23) (end 126.54 116.5) (width 0.2) (layer "F.Cu") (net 6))
 (segment (start 145.888135 142) (end 149.5 138.388135) (width 0.2) (layer "F.Cu") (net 6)))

